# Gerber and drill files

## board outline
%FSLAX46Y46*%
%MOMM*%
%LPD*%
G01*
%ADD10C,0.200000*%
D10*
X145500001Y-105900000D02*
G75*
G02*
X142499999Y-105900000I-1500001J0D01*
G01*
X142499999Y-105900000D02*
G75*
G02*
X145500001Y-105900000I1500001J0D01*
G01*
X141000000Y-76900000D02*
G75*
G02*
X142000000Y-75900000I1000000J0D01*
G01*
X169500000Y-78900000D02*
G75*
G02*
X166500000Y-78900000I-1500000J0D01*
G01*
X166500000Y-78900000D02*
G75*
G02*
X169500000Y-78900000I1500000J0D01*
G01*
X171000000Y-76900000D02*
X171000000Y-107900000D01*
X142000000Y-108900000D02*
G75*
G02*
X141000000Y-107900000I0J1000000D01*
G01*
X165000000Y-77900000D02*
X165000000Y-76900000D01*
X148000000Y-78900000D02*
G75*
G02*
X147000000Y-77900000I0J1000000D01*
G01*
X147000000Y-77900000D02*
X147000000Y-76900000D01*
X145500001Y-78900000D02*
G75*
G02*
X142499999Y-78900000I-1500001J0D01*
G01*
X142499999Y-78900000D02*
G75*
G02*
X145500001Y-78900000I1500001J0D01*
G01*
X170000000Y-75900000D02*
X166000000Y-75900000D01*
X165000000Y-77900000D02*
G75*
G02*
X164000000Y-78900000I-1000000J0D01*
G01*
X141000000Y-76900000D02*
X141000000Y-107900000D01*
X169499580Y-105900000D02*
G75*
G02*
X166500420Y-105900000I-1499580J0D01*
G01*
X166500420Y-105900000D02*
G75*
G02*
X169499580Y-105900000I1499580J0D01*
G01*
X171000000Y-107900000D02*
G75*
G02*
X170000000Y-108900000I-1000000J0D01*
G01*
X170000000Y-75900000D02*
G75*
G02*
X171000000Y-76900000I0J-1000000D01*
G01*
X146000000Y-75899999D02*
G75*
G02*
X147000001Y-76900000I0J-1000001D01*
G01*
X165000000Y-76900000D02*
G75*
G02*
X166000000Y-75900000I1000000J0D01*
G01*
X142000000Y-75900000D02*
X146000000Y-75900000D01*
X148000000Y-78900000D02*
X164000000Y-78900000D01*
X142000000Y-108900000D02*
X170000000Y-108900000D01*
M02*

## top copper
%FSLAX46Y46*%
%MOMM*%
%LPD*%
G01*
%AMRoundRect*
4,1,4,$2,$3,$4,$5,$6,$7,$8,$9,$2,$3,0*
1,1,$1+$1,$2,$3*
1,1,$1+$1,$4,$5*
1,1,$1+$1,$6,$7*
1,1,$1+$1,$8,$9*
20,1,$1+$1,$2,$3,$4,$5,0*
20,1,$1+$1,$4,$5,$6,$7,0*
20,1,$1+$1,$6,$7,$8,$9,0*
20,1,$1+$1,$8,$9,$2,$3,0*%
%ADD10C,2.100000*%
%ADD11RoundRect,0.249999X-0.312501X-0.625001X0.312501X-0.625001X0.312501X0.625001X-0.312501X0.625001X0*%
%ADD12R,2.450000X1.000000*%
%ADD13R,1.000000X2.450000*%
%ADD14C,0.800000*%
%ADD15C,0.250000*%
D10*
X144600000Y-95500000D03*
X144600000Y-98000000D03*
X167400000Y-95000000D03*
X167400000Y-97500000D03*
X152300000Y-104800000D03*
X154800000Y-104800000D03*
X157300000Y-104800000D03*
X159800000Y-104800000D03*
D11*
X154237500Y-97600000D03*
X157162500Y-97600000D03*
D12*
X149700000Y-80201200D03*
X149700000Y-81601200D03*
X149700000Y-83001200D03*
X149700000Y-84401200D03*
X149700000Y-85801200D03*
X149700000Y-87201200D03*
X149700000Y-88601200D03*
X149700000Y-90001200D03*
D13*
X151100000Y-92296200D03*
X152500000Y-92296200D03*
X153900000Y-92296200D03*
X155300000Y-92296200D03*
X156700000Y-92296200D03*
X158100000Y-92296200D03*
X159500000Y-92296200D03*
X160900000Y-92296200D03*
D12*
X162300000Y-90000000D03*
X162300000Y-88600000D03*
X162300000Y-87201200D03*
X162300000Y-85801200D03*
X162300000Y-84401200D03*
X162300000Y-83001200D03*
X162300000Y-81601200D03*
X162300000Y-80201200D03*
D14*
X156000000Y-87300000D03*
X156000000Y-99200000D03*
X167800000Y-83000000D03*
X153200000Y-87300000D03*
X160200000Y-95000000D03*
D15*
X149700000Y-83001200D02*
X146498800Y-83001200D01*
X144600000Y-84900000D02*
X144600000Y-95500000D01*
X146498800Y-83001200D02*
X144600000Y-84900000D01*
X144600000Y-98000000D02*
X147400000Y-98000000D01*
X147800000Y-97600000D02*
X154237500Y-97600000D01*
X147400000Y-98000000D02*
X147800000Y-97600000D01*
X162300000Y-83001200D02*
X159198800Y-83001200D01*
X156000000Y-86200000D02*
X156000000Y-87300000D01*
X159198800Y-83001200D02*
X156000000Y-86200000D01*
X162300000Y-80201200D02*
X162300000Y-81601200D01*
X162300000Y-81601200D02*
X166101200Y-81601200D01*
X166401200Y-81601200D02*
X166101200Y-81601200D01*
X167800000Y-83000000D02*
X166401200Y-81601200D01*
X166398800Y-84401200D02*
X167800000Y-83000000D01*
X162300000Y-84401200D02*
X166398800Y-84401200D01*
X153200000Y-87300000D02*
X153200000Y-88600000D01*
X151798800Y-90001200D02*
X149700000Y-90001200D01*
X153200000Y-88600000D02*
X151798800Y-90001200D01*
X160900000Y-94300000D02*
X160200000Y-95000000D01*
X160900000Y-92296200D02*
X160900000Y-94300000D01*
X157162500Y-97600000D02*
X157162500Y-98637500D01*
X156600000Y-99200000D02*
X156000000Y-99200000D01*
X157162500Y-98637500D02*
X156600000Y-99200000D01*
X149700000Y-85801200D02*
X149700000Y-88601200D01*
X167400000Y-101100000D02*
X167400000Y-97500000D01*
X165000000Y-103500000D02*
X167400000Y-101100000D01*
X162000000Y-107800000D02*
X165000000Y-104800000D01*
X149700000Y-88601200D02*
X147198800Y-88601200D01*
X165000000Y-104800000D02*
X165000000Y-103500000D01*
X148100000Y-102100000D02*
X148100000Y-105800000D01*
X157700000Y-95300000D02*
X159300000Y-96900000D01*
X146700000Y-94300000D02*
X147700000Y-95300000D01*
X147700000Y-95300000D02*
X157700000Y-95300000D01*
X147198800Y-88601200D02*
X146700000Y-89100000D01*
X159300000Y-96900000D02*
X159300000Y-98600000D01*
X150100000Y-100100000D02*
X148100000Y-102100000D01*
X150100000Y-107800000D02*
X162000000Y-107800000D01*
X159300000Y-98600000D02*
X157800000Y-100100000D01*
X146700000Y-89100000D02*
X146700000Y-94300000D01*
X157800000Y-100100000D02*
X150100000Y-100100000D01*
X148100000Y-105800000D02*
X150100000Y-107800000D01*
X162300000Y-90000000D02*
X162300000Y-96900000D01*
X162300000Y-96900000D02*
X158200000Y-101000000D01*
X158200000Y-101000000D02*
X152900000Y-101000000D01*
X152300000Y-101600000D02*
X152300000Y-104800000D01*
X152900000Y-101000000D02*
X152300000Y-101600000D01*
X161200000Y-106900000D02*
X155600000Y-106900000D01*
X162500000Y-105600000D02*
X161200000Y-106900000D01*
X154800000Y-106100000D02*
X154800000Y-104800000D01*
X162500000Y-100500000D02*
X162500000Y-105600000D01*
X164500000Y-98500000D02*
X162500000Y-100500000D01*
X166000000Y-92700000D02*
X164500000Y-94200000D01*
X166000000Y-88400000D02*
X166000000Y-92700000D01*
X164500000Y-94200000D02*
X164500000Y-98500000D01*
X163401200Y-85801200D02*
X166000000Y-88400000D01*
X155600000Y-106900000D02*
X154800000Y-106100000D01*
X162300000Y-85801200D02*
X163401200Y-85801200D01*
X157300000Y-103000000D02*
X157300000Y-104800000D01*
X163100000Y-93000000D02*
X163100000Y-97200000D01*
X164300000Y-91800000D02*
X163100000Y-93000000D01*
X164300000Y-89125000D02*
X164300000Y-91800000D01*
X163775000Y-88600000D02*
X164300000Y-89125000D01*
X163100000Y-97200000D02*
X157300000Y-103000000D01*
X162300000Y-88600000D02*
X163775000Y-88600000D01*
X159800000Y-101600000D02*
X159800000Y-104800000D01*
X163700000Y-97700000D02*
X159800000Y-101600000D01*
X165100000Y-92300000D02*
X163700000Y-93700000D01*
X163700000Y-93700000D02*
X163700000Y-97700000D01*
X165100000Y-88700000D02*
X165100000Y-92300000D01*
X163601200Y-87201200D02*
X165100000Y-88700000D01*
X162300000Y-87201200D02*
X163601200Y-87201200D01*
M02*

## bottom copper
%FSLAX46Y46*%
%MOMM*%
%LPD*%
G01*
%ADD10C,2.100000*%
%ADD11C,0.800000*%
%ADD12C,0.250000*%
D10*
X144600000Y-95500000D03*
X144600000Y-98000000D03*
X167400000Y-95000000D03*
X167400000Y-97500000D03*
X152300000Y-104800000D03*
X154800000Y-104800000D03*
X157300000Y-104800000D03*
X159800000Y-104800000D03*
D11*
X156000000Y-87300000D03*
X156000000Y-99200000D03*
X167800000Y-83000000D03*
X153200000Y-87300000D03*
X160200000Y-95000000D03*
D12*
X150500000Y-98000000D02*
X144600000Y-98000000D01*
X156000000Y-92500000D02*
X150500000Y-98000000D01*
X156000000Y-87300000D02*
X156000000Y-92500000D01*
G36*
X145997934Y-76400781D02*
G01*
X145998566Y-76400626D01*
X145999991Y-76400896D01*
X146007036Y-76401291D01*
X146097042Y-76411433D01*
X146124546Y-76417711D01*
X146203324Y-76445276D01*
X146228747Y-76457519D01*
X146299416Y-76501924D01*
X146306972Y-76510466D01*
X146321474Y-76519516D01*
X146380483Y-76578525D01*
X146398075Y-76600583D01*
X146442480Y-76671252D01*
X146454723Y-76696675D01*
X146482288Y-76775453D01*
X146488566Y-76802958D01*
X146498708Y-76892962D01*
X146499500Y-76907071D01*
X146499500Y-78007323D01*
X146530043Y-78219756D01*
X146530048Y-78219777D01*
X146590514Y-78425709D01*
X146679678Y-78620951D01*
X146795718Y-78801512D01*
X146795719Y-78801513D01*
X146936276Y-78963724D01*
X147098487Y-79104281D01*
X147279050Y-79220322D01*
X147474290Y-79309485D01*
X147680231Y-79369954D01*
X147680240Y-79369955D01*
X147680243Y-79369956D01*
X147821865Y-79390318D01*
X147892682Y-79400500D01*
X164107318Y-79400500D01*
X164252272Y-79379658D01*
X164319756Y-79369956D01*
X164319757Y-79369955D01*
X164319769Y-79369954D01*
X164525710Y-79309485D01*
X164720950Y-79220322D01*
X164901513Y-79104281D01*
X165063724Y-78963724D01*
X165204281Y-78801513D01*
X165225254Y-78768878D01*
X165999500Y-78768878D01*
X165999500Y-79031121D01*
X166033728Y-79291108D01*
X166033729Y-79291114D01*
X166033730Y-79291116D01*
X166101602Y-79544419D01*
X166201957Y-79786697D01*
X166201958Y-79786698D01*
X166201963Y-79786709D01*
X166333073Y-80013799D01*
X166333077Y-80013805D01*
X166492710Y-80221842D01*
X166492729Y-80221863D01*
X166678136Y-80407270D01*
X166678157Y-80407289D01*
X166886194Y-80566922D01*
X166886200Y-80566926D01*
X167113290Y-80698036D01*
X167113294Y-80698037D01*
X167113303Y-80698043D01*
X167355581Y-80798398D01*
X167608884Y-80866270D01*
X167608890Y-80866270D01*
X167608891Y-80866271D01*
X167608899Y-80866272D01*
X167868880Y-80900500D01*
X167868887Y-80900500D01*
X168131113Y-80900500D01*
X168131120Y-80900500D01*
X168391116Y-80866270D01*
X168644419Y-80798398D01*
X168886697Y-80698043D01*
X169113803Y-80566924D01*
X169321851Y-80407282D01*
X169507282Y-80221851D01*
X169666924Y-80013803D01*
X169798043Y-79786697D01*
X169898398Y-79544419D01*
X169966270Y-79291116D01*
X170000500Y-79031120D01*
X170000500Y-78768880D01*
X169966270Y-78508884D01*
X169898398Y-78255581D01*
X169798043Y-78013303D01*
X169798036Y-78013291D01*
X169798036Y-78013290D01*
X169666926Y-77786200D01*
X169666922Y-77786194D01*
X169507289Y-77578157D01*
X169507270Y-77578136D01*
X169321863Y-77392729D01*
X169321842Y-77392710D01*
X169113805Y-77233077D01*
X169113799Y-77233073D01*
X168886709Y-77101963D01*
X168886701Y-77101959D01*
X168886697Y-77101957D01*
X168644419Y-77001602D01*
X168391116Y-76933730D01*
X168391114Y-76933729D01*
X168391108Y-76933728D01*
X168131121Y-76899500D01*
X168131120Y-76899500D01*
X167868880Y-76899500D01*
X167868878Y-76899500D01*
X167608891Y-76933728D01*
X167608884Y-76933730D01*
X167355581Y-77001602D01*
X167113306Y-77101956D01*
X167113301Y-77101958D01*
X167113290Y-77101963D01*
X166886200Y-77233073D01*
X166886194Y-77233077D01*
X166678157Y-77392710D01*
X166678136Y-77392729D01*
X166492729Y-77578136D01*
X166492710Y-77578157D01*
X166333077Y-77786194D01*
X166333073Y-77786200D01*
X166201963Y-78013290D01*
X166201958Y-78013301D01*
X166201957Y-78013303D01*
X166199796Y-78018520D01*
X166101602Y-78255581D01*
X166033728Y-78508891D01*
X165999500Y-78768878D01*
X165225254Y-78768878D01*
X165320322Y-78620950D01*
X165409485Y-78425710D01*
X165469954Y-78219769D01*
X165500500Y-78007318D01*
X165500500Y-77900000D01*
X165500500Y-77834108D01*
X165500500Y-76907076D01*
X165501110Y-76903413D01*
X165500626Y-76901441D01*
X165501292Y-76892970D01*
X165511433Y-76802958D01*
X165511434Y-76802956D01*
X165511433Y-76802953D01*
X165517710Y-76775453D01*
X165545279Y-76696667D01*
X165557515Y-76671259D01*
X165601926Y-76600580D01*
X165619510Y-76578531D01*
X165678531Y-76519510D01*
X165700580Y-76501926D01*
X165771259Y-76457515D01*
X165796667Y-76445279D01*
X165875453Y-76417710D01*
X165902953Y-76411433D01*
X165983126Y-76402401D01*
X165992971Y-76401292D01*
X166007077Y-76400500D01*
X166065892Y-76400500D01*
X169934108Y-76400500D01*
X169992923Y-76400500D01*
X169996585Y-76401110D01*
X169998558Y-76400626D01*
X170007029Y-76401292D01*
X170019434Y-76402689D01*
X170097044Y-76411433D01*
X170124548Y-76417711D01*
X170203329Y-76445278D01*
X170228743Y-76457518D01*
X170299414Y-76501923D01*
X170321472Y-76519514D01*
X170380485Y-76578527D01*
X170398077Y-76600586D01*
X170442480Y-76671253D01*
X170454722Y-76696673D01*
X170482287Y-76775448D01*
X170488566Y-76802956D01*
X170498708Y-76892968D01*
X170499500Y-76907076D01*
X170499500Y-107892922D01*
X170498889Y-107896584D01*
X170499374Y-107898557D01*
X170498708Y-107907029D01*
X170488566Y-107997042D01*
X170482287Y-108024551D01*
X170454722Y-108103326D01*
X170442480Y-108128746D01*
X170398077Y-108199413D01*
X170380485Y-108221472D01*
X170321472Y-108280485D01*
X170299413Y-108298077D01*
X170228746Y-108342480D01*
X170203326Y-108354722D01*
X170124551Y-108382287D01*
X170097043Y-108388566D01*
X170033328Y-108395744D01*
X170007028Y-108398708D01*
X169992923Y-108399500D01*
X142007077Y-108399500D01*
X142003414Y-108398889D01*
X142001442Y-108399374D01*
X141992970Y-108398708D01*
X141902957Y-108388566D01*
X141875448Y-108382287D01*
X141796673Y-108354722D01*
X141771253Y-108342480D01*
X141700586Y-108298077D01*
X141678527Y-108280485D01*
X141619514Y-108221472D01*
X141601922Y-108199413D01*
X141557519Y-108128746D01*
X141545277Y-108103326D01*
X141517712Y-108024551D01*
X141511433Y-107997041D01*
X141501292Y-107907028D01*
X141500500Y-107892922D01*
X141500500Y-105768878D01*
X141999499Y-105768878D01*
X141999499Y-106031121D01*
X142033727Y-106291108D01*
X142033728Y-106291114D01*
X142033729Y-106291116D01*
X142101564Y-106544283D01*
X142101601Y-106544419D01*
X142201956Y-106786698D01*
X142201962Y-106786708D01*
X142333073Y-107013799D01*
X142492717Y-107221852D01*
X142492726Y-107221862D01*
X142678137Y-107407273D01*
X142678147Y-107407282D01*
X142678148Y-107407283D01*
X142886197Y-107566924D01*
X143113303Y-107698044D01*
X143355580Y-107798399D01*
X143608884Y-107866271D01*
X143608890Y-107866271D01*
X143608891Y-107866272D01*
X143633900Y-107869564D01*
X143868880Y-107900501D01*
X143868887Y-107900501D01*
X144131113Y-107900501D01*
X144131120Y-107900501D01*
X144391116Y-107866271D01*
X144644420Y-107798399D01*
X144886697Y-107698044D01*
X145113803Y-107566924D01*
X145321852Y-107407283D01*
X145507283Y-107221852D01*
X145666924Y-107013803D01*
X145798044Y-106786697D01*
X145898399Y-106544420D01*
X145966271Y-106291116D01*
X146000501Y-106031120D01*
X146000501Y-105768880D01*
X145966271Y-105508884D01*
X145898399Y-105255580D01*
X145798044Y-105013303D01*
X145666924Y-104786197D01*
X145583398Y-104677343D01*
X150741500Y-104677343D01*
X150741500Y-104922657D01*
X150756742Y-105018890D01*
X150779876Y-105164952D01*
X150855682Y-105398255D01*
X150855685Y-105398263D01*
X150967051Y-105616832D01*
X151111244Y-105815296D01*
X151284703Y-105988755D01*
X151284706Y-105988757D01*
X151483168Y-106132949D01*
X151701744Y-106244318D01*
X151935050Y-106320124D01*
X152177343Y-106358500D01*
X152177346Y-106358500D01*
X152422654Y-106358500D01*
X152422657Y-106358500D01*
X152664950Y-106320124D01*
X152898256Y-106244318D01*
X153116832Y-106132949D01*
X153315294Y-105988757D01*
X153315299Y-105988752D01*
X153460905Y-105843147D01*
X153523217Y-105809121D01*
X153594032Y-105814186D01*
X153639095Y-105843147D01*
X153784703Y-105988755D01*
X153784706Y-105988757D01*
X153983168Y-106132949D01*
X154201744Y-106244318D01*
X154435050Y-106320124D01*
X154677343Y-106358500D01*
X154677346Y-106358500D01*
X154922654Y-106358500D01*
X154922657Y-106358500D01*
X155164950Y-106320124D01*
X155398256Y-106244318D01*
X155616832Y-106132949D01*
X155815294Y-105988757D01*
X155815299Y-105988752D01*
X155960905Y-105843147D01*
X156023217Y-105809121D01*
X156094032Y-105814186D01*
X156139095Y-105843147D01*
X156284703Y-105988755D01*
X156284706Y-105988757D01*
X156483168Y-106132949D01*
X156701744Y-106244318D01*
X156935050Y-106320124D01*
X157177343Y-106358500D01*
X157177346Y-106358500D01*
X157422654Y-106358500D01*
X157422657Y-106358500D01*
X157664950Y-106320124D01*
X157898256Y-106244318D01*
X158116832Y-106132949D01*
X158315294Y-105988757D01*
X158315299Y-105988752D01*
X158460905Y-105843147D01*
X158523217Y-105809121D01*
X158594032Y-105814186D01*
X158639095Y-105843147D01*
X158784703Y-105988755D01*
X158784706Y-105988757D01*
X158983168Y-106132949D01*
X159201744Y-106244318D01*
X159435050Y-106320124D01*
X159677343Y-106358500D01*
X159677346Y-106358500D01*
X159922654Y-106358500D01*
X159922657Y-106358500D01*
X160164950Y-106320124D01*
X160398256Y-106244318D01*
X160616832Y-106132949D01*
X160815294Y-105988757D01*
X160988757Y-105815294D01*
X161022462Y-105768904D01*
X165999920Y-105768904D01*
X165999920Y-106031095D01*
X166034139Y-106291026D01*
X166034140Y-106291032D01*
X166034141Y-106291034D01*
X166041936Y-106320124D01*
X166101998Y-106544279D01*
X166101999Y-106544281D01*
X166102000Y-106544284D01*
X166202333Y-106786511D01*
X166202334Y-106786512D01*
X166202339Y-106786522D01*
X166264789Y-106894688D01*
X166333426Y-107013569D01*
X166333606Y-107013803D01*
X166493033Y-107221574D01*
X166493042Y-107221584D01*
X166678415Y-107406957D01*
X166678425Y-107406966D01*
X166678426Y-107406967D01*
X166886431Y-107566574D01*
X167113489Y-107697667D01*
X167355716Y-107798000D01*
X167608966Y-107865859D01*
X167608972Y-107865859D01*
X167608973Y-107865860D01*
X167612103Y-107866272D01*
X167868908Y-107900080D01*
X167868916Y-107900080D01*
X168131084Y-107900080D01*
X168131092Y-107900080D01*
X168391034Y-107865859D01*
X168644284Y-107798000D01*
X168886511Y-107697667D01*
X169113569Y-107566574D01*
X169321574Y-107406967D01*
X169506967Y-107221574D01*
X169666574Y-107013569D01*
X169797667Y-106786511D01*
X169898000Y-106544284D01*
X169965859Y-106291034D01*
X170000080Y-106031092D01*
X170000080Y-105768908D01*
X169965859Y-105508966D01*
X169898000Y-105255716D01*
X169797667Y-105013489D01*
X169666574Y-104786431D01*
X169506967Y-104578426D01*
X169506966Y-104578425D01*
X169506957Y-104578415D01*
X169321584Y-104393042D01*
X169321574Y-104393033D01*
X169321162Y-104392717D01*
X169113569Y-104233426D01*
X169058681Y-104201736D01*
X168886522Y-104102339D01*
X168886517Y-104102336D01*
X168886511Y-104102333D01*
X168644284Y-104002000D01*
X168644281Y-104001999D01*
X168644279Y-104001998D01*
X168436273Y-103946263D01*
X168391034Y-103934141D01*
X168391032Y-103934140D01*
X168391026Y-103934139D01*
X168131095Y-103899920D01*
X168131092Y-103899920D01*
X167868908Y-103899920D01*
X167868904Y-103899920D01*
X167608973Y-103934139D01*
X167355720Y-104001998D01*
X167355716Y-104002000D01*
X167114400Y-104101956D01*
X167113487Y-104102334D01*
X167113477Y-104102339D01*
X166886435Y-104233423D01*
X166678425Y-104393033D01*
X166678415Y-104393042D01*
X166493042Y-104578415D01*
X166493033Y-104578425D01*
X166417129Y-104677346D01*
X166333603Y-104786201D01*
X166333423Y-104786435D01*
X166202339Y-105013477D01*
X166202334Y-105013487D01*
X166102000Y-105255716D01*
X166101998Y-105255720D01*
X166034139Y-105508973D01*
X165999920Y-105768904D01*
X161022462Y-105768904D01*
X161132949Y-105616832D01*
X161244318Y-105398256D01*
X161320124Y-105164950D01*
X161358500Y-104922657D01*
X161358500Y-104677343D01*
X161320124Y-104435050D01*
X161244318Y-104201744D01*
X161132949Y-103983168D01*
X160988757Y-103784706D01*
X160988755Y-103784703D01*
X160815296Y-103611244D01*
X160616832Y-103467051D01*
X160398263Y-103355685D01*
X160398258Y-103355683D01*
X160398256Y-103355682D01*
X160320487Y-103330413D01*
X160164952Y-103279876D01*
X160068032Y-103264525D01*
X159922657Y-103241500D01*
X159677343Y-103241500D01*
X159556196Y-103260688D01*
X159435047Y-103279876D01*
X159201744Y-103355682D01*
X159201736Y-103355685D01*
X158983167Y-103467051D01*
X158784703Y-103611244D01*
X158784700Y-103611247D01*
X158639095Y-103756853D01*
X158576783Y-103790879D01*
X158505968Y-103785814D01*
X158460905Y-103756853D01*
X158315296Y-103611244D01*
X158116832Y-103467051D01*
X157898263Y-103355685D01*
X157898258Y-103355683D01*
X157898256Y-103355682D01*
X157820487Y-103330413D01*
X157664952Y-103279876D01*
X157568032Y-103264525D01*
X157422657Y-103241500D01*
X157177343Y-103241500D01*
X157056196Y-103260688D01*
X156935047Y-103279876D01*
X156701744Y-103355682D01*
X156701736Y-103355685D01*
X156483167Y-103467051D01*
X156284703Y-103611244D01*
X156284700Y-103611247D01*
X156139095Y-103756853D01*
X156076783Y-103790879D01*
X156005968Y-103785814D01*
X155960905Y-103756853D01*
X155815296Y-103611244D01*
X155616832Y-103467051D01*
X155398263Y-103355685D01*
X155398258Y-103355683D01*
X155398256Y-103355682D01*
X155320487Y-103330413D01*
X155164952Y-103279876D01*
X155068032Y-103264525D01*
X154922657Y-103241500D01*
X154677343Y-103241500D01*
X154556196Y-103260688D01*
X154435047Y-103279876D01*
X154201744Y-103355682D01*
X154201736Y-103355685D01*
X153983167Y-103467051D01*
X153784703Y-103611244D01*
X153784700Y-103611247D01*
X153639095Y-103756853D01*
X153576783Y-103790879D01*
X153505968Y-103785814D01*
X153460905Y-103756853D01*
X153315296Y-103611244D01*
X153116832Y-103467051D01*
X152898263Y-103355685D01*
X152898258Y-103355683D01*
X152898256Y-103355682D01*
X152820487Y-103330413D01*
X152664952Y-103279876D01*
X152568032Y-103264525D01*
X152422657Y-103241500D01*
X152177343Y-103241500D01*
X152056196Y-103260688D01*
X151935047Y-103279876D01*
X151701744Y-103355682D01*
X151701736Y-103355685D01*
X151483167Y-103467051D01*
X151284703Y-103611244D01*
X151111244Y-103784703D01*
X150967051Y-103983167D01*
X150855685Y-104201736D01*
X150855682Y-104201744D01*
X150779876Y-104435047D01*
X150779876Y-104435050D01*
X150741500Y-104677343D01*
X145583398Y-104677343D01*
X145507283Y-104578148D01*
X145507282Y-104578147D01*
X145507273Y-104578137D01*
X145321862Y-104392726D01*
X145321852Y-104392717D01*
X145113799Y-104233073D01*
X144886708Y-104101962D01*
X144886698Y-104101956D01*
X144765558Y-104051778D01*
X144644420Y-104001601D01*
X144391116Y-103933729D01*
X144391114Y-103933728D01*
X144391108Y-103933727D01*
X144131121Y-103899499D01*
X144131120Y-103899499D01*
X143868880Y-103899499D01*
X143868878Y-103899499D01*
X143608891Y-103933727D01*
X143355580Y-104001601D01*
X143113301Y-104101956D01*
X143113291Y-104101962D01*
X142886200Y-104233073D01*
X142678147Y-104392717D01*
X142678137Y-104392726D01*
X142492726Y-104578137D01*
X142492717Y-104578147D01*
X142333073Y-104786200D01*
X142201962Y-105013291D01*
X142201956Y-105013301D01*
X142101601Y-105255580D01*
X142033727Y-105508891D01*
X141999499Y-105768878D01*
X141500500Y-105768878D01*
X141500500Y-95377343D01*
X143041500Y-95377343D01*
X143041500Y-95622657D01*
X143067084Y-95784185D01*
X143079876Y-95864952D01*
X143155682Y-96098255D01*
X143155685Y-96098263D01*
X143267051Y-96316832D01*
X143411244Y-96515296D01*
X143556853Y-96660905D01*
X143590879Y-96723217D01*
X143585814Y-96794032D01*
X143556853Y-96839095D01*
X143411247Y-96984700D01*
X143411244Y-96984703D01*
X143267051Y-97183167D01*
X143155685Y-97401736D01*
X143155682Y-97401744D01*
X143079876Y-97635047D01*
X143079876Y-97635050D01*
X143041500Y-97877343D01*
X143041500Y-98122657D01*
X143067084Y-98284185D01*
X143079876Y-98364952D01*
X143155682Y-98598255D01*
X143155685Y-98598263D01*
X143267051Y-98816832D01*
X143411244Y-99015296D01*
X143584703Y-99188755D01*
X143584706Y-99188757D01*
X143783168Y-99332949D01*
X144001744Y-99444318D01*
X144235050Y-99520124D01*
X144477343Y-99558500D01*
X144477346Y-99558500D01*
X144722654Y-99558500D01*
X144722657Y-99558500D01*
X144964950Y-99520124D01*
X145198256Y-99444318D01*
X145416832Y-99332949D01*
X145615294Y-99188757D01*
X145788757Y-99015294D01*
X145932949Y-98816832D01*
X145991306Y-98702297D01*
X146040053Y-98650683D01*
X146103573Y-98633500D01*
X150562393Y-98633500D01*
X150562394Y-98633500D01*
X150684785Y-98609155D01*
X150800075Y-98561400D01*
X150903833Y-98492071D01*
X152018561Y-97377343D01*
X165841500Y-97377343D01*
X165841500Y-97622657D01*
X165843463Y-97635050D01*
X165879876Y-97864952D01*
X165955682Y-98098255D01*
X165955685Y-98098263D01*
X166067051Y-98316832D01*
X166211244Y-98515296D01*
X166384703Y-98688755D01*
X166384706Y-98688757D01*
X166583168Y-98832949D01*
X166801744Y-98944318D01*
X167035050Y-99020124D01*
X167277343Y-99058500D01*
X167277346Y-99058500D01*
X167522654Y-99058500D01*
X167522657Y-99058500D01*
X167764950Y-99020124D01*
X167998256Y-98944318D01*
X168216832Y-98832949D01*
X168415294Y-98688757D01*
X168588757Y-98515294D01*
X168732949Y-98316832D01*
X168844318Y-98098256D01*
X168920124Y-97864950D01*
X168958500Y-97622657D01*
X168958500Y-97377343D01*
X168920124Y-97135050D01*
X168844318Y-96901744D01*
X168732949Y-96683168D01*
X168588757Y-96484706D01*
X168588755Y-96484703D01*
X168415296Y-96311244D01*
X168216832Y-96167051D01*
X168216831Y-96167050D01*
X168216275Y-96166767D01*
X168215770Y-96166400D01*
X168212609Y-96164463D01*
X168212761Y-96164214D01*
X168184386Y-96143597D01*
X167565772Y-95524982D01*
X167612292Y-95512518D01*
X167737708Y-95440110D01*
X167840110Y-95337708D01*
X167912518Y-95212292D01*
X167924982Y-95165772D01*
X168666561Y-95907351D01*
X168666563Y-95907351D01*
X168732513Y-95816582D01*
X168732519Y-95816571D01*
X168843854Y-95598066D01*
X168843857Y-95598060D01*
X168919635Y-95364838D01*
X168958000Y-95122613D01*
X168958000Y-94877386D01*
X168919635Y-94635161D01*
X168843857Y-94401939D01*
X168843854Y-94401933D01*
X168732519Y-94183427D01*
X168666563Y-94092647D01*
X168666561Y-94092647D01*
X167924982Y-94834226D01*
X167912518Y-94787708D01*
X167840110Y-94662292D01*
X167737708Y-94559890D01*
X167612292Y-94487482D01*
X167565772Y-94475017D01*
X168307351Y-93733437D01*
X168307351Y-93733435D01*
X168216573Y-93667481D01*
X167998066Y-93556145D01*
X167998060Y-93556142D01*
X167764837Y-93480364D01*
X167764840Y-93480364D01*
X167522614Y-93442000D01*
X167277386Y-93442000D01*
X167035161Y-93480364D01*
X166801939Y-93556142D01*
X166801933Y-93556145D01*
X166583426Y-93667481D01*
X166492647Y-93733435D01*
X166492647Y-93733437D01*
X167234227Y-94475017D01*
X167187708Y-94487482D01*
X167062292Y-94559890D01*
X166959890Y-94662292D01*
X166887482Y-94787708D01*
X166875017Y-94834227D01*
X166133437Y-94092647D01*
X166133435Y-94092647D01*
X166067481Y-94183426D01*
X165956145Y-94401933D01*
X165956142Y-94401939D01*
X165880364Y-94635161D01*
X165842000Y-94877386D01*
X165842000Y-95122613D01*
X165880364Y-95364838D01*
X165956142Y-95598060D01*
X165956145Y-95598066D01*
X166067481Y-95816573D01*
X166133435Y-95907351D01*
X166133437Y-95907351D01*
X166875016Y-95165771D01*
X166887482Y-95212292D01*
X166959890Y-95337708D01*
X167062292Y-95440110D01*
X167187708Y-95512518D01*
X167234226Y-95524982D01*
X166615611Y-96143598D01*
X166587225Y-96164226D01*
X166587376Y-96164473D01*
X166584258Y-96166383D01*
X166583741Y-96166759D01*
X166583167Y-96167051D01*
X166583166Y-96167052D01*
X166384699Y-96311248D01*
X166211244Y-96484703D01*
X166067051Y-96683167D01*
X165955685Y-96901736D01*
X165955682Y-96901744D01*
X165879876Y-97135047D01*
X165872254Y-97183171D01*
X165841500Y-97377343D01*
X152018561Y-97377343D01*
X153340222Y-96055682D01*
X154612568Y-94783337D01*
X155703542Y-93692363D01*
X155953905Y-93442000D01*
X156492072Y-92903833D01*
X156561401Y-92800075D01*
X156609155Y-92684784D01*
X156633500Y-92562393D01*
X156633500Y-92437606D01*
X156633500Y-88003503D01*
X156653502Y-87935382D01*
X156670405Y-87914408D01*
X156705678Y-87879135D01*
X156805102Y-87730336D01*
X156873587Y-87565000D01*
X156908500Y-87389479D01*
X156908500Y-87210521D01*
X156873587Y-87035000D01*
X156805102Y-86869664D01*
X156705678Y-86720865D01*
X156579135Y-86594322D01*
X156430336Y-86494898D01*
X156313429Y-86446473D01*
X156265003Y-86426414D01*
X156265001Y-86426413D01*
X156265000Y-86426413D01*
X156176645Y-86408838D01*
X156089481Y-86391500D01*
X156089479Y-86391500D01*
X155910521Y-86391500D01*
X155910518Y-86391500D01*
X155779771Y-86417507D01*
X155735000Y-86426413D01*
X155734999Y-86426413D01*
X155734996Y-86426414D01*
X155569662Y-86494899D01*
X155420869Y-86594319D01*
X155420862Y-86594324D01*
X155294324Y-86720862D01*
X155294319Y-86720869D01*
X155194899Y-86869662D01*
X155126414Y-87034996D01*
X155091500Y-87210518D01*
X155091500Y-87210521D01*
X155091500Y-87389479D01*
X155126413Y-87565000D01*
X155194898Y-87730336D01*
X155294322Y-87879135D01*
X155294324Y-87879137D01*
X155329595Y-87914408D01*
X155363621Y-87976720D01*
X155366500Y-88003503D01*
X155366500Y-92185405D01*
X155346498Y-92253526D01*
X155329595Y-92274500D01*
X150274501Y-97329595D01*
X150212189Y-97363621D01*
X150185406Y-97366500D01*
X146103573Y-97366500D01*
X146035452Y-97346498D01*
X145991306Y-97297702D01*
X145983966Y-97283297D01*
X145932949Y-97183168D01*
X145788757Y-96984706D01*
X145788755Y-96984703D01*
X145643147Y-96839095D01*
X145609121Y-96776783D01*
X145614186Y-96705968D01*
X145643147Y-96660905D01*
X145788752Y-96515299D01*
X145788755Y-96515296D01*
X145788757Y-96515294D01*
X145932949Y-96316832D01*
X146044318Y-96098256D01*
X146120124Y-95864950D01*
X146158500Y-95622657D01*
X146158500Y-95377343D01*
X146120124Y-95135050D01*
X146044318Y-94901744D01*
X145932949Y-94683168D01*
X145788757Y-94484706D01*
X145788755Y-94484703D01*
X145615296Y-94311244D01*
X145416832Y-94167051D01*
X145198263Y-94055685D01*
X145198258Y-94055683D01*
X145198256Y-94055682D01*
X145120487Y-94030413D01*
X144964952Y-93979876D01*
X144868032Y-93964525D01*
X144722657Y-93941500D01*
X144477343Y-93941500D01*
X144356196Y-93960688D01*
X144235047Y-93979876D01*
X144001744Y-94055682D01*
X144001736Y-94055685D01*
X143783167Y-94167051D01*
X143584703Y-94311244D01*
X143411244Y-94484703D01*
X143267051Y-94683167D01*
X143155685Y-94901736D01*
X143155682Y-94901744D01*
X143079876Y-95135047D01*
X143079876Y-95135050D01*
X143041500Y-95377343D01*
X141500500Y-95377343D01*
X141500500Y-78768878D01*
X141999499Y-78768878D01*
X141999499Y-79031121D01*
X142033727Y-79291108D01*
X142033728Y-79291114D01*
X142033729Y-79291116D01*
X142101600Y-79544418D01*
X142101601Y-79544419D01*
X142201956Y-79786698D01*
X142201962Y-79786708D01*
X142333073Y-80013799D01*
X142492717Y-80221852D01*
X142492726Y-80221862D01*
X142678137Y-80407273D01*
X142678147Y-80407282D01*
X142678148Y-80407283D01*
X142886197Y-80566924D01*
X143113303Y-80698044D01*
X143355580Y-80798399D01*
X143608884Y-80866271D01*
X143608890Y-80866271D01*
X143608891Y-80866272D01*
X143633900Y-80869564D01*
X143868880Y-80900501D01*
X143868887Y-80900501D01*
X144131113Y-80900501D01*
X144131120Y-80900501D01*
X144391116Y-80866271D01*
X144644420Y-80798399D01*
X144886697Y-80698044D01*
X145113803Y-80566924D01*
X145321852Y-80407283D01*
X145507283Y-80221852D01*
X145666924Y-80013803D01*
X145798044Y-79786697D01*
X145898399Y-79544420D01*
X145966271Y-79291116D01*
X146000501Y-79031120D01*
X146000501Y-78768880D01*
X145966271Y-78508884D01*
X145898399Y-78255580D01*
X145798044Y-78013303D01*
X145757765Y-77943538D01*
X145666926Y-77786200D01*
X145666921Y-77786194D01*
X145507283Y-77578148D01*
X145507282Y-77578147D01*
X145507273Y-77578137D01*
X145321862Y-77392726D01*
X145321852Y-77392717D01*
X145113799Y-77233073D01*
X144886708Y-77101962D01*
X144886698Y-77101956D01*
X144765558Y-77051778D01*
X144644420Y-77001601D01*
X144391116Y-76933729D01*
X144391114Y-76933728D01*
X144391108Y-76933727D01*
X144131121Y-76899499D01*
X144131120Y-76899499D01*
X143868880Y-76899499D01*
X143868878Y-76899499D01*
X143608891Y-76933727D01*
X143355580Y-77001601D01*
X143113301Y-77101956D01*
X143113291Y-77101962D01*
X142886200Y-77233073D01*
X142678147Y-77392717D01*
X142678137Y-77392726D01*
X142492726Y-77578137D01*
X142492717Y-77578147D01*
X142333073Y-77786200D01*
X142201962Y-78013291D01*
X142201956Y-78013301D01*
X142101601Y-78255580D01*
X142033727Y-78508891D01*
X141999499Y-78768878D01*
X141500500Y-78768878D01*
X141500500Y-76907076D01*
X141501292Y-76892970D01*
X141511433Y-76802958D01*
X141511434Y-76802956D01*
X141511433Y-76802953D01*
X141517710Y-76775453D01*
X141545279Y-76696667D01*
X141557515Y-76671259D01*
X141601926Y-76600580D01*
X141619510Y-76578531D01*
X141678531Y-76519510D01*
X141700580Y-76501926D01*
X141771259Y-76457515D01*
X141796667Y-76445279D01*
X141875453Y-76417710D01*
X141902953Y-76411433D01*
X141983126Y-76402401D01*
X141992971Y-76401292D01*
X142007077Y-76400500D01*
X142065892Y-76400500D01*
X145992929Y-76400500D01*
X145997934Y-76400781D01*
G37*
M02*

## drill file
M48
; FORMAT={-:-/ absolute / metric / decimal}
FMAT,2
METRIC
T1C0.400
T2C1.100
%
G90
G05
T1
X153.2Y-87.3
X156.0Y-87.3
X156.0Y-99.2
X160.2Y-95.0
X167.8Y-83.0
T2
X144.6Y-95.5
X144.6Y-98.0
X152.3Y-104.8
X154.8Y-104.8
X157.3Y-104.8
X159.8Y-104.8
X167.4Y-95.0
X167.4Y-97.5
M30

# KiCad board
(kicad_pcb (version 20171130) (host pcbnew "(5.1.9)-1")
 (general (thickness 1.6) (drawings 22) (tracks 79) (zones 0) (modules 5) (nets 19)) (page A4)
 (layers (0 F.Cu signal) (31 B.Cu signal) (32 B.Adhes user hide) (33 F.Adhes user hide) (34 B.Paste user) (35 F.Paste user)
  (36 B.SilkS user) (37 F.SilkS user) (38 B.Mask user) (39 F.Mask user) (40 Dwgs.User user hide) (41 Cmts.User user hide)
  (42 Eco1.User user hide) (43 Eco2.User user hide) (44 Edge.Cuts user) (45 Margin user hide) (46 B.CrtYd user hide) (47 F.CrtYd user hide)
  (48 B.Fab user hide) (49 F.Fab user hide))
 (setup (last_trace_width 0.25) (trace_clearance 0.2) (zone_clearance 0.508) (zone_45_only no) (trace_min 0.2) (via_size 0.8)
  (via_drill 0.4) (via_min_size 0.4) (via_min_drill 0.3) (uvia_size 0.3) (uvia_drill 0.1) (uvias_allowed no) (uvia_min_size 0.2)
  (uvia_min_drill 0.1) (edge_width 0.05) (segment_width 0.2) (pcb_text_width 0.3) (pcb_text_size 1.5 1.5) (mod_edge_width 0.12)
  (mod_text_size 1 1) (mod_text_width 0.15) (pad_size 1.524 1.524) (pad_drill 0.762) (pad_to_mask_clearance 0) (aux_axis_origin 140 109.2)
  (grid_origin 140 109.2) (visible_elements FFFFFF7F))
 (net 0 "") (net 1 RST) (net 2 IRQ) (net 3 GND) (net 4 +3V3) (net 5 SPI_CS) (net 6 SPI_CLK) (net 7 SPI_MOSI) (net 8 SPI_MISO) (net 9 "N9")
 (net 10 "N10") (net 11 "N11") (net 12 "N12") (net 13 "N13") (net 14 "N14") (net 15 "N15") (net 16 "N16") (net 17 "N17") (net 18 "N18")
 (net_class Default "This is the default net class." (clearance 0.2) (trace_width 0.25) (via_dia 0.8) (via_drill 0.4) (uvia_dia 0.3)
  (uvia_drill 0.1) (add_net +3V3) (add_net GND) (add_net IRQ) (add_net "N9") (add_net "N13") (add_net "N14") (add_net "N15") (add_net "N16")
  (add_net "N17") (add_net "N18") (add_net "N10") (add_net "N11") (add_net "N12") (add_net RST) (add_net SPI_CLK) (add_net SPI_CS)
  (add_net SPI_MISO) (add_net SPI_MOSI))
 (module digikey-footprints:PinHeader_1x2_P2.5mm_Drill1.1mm (layer F.Cu) (at 144.6 98 90)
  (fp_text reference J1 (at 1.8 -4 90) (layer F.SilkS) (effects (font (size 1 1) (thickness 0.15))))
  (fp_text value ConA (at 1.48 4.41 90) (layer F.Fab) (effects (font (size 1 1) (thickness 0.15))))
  (pad 2 thru_hole circle (at 2.5 0 90) (size 2.1 2.1) (drill 1.1) (layers *.Cu *.Mask) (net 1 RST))
  (pad 1 thru_hole circle (at 0 0 90) (size 2.1 2.1) (drill 1.1) (layers *.Cu *.Mask) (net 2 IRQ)))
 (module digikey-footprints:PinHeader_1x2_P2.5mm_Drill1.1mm (layer F.Cu) (at 167.4 95 270)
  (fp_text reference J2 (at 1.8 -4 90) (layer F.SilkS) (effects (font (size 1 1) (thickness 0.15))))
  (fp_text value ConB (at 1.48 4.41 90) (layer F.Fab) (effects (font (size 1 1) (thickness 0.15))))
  (pad 1 thru_hole circle (at 0 0 270) (size 2.1 2.1) (drill 1.1) (layers *.Cu *.Mask) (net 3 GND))
  (pad 2 thru_hole circle (at 2.5 0 270) (size 2.1 2.1) (drill 1.1) (layers *.Cu *.Mask) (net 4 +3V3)))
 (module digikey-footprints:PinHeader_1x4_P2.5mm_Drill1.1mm (layer F.Cu) (at 152.3 104.8)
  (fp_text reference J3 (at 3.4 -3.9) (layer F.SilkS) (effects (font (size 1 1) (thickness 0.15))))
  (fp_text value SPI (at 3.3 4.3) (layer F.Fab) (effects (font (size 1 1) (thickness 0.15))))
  (pad 1 thru_hole circle (at 0 0) (size 2.1 2.1) (drill 1.1) (layers *.Cu *.Mask) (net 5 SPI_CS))
  (pad 2 thru_hole circle (at 2.5 0) (size 2.1 2.1) (drill 1.1) (layers *.Cu *.Mask) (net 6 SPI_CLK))
  (pad 3 thru_hole circle (at 5 0) (size 2.1 2.1) (drill 1.1) (layers *.Cu *.Mask) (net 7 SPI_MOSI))
  (pad 4 thru_hole circle (at 7.5 0) (size 2.1 2.1) (drill 1.1) (layers *.Cu *.Mask) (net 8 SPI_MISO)))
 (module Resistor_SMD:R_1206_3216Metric (layer F.Cu) (at 155.7 97.6)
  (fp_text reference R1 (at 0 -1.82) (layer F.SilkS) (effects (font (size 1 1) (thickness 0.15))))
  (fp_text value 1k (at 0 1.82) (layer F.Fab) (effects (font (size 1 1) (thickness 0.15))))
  (pad 1 smd roundrect (at -1.4625 0) (size 1.125 1.75) (layers F.Cu F.Paste F.Mask) (roundrect_rratio 0.2222213333333333) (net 2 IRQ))
  (pad 2 smd roundrect (at 1.4625 0) (size 1.125 1.75) (layers F.Cu F.Paste F.Mask) (roundrect_rratio 0.2222213333333333) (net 3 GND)))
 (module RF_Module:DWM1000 (layer F.Cu) (at 156 81)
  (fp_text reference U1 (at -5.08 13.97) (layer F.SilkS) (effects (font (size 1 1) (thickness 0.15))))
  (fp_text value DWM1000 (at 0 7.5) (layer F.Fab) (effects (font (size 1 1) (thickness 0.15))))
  (pad 1 smd rect (at -6.3 -0.7988 90) (size 1 2.45) (layers F.Cu F.Paste F.Mask) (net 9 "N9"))
  (pad 2 smd rect (at -6.3 0.6012 90) (size 1 2.45) (layers F.Cu F.Paste F.Mask) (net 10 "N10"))
  (pad 3 smd rect (at -6.3 2.0012 90) (size 1 2.45) (layers F.Cu F.Paste F.Mask) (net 1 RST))
  (pad 4 smd rect (at -6.3 3.4012 90) (size 1 2.45) (layers F.Cu F.Paste F.Mask) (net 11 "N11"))
  (pad 5 smd rect (at -6.3 4.8012 90) (size 1 2.45) (layers F.Cu F.Paste F.Mask) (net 4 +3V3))
  (pad 6 smd rect (at -6.3 6.2012 90) (size 1 2.45) (layers F.Cu F.Paste F.Mask) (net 4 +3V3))
  (pad 7 smd rect (at -6.3 7.6012 90) (size 1 2.45) (layers F.Cu F.Paste F.Mask) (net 4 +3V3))
  (pad 8 smd rect (at -6.3 9.0012 90) (size 1 2.45) (layers F.Cu F.Paste F.Mask) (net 3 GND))
  (pad 9 smd rect (at -4.9 11.2962) (size 1 2.45) (layers F.Cu F.Paste F.Mask) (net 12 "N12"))
  (pad 10 smd rect (at -3.5 11.2962) (size 1 2.45) (layers F.Cu F.Paste F.Mask) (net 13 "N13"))
  (pad 11 smd rect (at -2.1 11.2962) (size 1 2.45) (layers F.Cu F.Paste F.Mask) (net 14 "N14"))
  (pad 12 smd rect (at -0.7 11.2962) (size 1 2.45) (layers F.Cu F.Paste F.Mask) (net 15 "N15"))
  (pad 13 smd rect (at 0.7 11.2962) (size 1 2.45) (layers F.Cu F.Paste F.Mask) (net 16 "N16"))
  (pad 14 smd rect (at 2.1 11.2962) (size 1 2.45) (layers F.Cu F.Paste F.Mask) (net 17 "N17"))
  (pad 15 smd rect (at 3.5 11.2962) (size 1 2.45) (layers F.Cu F.Paste F.Mask) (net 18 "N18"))
  (pad 16 smd rect (at 4.9 11.2962) (size 1 2.45) (layers F.Cu F.Paste F.Mask) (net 3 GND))
  (pad 17 smd rect (at 6.3 9 90) (size 1 2.45) (layers F.Cu F.Paste F.Mask) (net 5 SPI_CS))
  (pad 18 smd rect (at 6.3 7.6 90) (size 1 2.45) (layers F.Cu F.Paste F.Mask) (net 7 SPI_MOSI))
  (pad 19 smd rect (at 6.3 6.2012 90) (size 1 2.45) (layers F.Cu F.Paste F.Mask) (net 8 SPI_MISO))
  (pad 20 smd rect (at 6.3 4.8012 90) (size 1 2.45) (layers F.Cu F.Paste F.Mask) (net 6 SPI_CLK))
  (pad 21 smd rect (at 6.3 3.4012 90) (size 1 2.45) (layers F.Cu F.Paste F.Mask) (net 3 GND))
  (pad 22 smd rect (at 6.3 2.0012 90) (size 1 2.45) (layers F.Cu F.Paste F.Mask) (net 2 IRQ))
  (pad 23 smd rect (at 6.3 0.6012 90) (size 1 2.45) (layers F.Cu F.Paste F.Mask) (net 3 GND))
  (pad 24 smd rect (at 6.3 -0.7988 90) (size 1 2.45) (layers F.Cu F.Paste F.Mask) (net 3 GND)))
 (gr_circle (center 144 105.9) (end 145.500001 105.9) (layer Edge.Cuts) (width 0.2))
 (gr_arc (start 142 76.9) (end 142 75.9) (angle -90) (layer Edge.Cuts) (width 0.2))
 (gr_circle (center 168 78.9) (end 169.5 78.9) (layer Edge.Cuts) (width 0.2))
 (gr_line (start 171 76.9) (end 171 107.9) (layer Edge.Cuts) (width 0.2))
 (gr_arc (start 142 107.9) (end 141 107.9) (angle -90) (layer Edge.Cuts) (width 0.2))
 (gr_line (start 165 77.9) (end 165 76.9) (layer Edge.Cuts) (width 0.2))
 (gr_arc (start 148 77.9) (end 147 77.9) (angle -90) (layer Edge.Cuts) (width 0.2))
 (gr_line (start 147 77.9) (end 147 76.9) (layer Edge.Cuts) (width 0.2))
 (gr_circle (center 144 78.9) (end 145.500001 78.9) (layer Edge.Cuts) (width 0.2))
 (gr_line (start 170 75.9) (end 166 75.9) (layer Edge.Cuts) (width 0.2))
 (gr_arc (start 164 77.9) (end 164 78.9) (angle -90) (layer Edge.Cuts) (width 0.2))
 (gr_line (start 141 76.9) (end 141 107.9) (layer Edge.Cuts) (width 0.2))
 (gr_circle (center 168 105.9) (end 169.49958 105.9) (layer Edge.Cuts) (width 0.2))
 (gr_arc (start 170 107.9) (end 170 108.9) (angle -90) (layer Edge.Cuts) (width 0.2))
 (gr_arc (start 170 76.9) (end 171 76.9) (angle -90) (layer Edge.Cuts) (width 0.2))
 (gr_arc (start 146 76.9) (end 147.000001 76.9) (angle -90) (layer Edge.Cuts) (width 0.2))
 (gr_arc (start 166 76.9) (end 166 75.9) (angle -90) (layer Edge.Cuts) (width 0.2))
 (gr_line (start 142 75.9) (end 146 75.9) (layer Edge.Cuts) (width 0.2))
 (gr_line (start 148 78.9) (end 164 78.9) (layer Edge.Cuts) (width 0.2))
 (gr_line (start 142 108.9) (end 170 108.9) (layer Edge.Cuts) (width 0.2))
 (via (at 156 87.3) (size 0.8) (drill 0.4) (layers F.Cu B.Cu) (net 2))
 (via (at 156 99.2) (size 0.8) (drill 0.4) (layers F.Cu B.Cu) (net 3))
 (segment (start 149.7 83.0012) (end 146.4988 83.0012) (width 0.25) (layer F.Cu) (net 1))
 (segment (start 144.6 84.9) (end 144.6 95.5) (width 0.25) (layer F.Cu) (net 1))
 (segment (start 146.4988 83.0012) (end 144.6 84.9) (width 0.25) (layer F.Cu) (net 1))
 (segment (start 144.6 98) (end 147.4 98) (width 0.25) (layer F.Cu) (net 2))
 (segment (start 147.8 97.6) (end 154.2375 97.6) (width 0.25) (layer F.Cu) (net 2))
 (segment (start 147.4 98) (end 147.8 97.6) (width 0.25) (layer F.Cu) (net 2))
 (segment (start 162.3 83.0012) (end 159.1988 83.0012) (width 0.25) (layer F.Cu) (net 2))
 (segment (start 156 86.2) (end 156 87.3) (width 0.25) (layer F.Cu) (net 2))
 (segment (start 159.1988 83.0012) (end 156 86.2) (width 0.25) (layer F.Cu) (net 2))
 (segment (start 150.5 98) (end 144.6 98) (width 0.25) (layer B.Cu) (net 2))
 (segment (start 156 92.5) (end 150.5 98) (width 0.25) (layer B.Cu) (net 2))
 (segment (start 156 87.3) (end 156 92.5) (width 0.25) (layer B.Cu) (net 2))
 (via (at 167.8 83) (size 0.8) (drill 0.4) (layers F.Cu B.Cu) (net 3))
 (via (at 153.2 87.3) (size 0.8) (drill 0.4) (layers F.Cu B.Cu) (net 3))
 (segment (start 162.3 80.2012) (end 162.3 81.6012) (width 0.25) (layer F.Cu) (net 3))
 (segment (start 162.3 81.6012) (end 166.1012 81.6012) (width 0.25) (layer F.Cu) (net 3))
 (segment (start 166.4012 81.6012) (end 166.1012 81.6012) (width 0.25) (layer F.Cu) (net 3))
 (segment (start 167.8 83) (end 166.4012 81.6012) (width 0.25) (layer F.Cu) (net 3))
 (segment (start 166.3988 84.4012) (end 167.8 83) (width 0.25) (layer F.Cu) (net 3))
 (segment (start 162.3 84.4012) (end 166.3988 84.4012) (width 0.25) (layer F.Cu) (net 3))
 (segment (start 153.2 87.3) (end 153.2 88.6) (width 0.25) (layer F.Cu) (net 3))
 (segment (start 151.7988 90.0012) (end 149.7 90.0012) (width 0.25) (layer F.Cu) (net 3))
 (segment (start 153.2 88.6) (end 151.7988 90.0012) (width 0.25) (layer F.Cu) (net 3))
 (via (at 160.2 95) (size 0.8) (drill 0.4) (layers F.Cu B.Cu) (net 3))
 (segment (start 160.9 94.3) (end 160.2 95) (width 0.25) (layer F.Cu) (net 3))
 (segment (start 160.9 92.2962) (end 160.9 94.3) (width 0.25) (layer F.Cu) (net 3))
 (segment (start 157.1625 97.6) (end 157.1625 98.6375) (width 0.25) (layer F.Cu) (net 3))
 (segment (start 156.6 99.2) (end 156 99.2) (width 0.25) (layer F.Cu) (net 3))
 (segment (start 157.1625 98.6375) (end 156.6 99.2) (width 0.25) (layer F.Cu) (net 3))
 (segment (start 149.7 85.8012) (end 149.7 88.6012) (width 0.25) (layer F.Cu) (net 4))
 (segment (start 167.4 101.1) (end 167.4 97.5) (width 0.25) (layer F.Cu) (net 4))
 (segment (start 165 103.5) (end 167.4 101.1) (width 0.25) (layer F.Cu) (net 4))
 (segment (start 162 107.8) (end 165 104.8) (width 0.25) (layer F.Cu) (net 4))
 (segment (start 149.7 88.6012) (end 147.1988 88.6012) (width 0.25) (layer F.Cu) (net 4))
 (segment (start 165 104.8) (end 165 103.5) (width 0.25) (layer F.Cu) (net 4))
 (segment (start 148.1 102.1) (end 148.1 105.8) (width 0.25) (layer F.Cu) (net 4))
 (segment (start 157.7 95.3) (end 159.3 96.9) (width 0.25) (layer F.Cu) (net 4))
 (segment (start 146.7 94.3) (end 147.7 95.3) (width 0.25) (layer F.Cu) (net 4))
 (segment (start 147.7 95.3) (end 157.7 95.3) (width 0.25) (layer F.Cu) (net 4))
 (segment (start 147.1988 88.6012) (end 146.7 89.1) (width 0.25) (layer F.Cu) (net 4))
 (segment (start 159.3 96.9) (end 159.3 98.6) (width 0.25) (layer F.Cu) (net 4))
 (segment (start 150.1 100.1) (end 148.1 102.1) (width 0.25) (layer F.Cu) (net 4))
 (segment (start 150.1 107.8) (end 162 107.8) (width 0.25) (layer F.Cu) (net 4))
 (segment (start 159.3 98.6) (end 157.8 100.1) (width 0.25) (layer F.Cu) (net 4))
 (segment (start 146.7 89.1) (end 146.7 94.3) (width 0.25) (layer F.Cu) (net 4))
 (segment (start 157.8 100.1) (end 150.1 100.1) (width 0.25) (layer F.Cu) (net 4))
 (segment (start 148.1 105.8) (end 150.1 107.8) (width 0.25) (layer F.Cu) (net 4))
 (segment (start 162.3 90) (end 162.3 96.9) (width 0.25) (layer F.Cu) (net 5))
 (segment (start 162.3 96.9) (end 158.2 101) (width 0.25) (layer F.Cu) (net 5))
 (segment (start 158.2 101) (end 152.9 101) (width 0.25) (layer F.Cu) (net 5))
 (segment (start 152.3 101.6) (end 152.3 104.8) (width 0.25) (layer F.Cu) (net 5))
 (segment (start 152.9 101) (end 152.3 101.6) (width 0.25) (layer F.Cu) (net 5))
 (segment (start 161.2 106.9) (end 155.6 106.9) (width 0.25) (layer F.Cu) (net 6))
 (segment (start 162.5 105.6) (end 161.2 106.9) (width 0.25) (layer F.Cu) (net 6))
 (segment (start 154.8 106.1) (end 154.8 104.8) (width 0.25) (layer F.Cu) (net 6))
 (segment (start 162.5 100.5) (end 162.5 105.6) (width 0.25) (layer F.Cu) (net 6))
 (segment (start 164.5 98.5) (end 162.5 100.5) (width 0.25) (layer F.Cu) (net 6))
 (segment (start 166 92.7) (end 164.5 94.2) (width 0.25) (layer F.Cu) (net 6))
 (segment (start 166 88.4) (end 166 92.7) (width 0.25) (layer F.Cu) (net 6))
 (segment (start 164.5 94.2) (end 164.5 98.5) (width 0.25) (layer F.Cu) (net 6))
 (segment (start 163.4012 85.8012) (end 166 88.4) (width 0.25) (layer F.Cu) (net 6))
 (segment (start 155.6 106.9) (end 154.8 106.1) (width 0.25) (layer F.Cu) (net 6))
 (segment (start 162.3 85.8012) (end 163.4012 85.8012) (width 0.25) (layer F.Cu) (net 6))
 (segment (start 157.3 103) (end 157.3 104.8) (width 0.25) (layer F.Cu) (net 7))
 (segment (start 163.1 93) (end 163.1 97.2) (width 0.25) (layer F.Cu) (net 7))
 (segment (start 164.3 91.8) (end 163.1 93) (width 0.25) (layer F.Cu) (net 7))
 (segment (start 164.3 89.125) (end 164.3 91.8) (width 0.25) (layer F.Cu) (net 7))
 (segment (start 163.775 88.6) (end 164.3 89.125) (width 0.25) (layer F.Cu) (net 7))
 (segment (start 163.1 97.2) (end 157.3 103) (width 0.25) (layer F.Cu) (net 7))
 (segment (start 162.3 88.6) (end 163.775 88.6) (width 0.25) (layer F.Cu) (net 7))
 (segment (start 159.8 101.6) (end 159.8 104.8) (width 0.25) (layer F.Cu) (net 8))
 (segment (start 163.7 97.7) (end 159.8 101.6) (width 0.25) (layer F.Cu) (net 8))
 (segment (start 165.1 92.3) (end 163.7 93.7) (width 0.25) (layer F.Cu) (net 8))
 (segment (start 163.7 93.7) (end 163.7 97.7) (width 0.25) (layer F.Cu) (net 8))
 (segment (start 165.1 88.7) (end 165.1 92.3) (width 0.25) (layer F.Cu) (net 8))
 (segment (start 163.6012 87.2012) (end 165.1 88.7) (width 0.25) (layer F.Cu) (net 8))
 (segment (start 162.3 87.2012) (end 163.6012 87.2012) (width 0.25) (layer F.Cu) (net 8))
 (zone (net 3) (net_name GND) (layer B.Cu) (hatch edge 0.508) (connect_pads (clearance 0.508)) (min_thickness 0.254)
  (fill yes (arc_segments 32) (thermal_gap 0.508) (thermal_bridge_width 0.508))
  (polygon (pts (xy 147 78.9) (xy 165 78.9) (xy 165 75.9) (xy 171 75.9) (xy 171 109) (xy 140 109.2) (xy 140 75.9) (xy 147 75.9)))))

